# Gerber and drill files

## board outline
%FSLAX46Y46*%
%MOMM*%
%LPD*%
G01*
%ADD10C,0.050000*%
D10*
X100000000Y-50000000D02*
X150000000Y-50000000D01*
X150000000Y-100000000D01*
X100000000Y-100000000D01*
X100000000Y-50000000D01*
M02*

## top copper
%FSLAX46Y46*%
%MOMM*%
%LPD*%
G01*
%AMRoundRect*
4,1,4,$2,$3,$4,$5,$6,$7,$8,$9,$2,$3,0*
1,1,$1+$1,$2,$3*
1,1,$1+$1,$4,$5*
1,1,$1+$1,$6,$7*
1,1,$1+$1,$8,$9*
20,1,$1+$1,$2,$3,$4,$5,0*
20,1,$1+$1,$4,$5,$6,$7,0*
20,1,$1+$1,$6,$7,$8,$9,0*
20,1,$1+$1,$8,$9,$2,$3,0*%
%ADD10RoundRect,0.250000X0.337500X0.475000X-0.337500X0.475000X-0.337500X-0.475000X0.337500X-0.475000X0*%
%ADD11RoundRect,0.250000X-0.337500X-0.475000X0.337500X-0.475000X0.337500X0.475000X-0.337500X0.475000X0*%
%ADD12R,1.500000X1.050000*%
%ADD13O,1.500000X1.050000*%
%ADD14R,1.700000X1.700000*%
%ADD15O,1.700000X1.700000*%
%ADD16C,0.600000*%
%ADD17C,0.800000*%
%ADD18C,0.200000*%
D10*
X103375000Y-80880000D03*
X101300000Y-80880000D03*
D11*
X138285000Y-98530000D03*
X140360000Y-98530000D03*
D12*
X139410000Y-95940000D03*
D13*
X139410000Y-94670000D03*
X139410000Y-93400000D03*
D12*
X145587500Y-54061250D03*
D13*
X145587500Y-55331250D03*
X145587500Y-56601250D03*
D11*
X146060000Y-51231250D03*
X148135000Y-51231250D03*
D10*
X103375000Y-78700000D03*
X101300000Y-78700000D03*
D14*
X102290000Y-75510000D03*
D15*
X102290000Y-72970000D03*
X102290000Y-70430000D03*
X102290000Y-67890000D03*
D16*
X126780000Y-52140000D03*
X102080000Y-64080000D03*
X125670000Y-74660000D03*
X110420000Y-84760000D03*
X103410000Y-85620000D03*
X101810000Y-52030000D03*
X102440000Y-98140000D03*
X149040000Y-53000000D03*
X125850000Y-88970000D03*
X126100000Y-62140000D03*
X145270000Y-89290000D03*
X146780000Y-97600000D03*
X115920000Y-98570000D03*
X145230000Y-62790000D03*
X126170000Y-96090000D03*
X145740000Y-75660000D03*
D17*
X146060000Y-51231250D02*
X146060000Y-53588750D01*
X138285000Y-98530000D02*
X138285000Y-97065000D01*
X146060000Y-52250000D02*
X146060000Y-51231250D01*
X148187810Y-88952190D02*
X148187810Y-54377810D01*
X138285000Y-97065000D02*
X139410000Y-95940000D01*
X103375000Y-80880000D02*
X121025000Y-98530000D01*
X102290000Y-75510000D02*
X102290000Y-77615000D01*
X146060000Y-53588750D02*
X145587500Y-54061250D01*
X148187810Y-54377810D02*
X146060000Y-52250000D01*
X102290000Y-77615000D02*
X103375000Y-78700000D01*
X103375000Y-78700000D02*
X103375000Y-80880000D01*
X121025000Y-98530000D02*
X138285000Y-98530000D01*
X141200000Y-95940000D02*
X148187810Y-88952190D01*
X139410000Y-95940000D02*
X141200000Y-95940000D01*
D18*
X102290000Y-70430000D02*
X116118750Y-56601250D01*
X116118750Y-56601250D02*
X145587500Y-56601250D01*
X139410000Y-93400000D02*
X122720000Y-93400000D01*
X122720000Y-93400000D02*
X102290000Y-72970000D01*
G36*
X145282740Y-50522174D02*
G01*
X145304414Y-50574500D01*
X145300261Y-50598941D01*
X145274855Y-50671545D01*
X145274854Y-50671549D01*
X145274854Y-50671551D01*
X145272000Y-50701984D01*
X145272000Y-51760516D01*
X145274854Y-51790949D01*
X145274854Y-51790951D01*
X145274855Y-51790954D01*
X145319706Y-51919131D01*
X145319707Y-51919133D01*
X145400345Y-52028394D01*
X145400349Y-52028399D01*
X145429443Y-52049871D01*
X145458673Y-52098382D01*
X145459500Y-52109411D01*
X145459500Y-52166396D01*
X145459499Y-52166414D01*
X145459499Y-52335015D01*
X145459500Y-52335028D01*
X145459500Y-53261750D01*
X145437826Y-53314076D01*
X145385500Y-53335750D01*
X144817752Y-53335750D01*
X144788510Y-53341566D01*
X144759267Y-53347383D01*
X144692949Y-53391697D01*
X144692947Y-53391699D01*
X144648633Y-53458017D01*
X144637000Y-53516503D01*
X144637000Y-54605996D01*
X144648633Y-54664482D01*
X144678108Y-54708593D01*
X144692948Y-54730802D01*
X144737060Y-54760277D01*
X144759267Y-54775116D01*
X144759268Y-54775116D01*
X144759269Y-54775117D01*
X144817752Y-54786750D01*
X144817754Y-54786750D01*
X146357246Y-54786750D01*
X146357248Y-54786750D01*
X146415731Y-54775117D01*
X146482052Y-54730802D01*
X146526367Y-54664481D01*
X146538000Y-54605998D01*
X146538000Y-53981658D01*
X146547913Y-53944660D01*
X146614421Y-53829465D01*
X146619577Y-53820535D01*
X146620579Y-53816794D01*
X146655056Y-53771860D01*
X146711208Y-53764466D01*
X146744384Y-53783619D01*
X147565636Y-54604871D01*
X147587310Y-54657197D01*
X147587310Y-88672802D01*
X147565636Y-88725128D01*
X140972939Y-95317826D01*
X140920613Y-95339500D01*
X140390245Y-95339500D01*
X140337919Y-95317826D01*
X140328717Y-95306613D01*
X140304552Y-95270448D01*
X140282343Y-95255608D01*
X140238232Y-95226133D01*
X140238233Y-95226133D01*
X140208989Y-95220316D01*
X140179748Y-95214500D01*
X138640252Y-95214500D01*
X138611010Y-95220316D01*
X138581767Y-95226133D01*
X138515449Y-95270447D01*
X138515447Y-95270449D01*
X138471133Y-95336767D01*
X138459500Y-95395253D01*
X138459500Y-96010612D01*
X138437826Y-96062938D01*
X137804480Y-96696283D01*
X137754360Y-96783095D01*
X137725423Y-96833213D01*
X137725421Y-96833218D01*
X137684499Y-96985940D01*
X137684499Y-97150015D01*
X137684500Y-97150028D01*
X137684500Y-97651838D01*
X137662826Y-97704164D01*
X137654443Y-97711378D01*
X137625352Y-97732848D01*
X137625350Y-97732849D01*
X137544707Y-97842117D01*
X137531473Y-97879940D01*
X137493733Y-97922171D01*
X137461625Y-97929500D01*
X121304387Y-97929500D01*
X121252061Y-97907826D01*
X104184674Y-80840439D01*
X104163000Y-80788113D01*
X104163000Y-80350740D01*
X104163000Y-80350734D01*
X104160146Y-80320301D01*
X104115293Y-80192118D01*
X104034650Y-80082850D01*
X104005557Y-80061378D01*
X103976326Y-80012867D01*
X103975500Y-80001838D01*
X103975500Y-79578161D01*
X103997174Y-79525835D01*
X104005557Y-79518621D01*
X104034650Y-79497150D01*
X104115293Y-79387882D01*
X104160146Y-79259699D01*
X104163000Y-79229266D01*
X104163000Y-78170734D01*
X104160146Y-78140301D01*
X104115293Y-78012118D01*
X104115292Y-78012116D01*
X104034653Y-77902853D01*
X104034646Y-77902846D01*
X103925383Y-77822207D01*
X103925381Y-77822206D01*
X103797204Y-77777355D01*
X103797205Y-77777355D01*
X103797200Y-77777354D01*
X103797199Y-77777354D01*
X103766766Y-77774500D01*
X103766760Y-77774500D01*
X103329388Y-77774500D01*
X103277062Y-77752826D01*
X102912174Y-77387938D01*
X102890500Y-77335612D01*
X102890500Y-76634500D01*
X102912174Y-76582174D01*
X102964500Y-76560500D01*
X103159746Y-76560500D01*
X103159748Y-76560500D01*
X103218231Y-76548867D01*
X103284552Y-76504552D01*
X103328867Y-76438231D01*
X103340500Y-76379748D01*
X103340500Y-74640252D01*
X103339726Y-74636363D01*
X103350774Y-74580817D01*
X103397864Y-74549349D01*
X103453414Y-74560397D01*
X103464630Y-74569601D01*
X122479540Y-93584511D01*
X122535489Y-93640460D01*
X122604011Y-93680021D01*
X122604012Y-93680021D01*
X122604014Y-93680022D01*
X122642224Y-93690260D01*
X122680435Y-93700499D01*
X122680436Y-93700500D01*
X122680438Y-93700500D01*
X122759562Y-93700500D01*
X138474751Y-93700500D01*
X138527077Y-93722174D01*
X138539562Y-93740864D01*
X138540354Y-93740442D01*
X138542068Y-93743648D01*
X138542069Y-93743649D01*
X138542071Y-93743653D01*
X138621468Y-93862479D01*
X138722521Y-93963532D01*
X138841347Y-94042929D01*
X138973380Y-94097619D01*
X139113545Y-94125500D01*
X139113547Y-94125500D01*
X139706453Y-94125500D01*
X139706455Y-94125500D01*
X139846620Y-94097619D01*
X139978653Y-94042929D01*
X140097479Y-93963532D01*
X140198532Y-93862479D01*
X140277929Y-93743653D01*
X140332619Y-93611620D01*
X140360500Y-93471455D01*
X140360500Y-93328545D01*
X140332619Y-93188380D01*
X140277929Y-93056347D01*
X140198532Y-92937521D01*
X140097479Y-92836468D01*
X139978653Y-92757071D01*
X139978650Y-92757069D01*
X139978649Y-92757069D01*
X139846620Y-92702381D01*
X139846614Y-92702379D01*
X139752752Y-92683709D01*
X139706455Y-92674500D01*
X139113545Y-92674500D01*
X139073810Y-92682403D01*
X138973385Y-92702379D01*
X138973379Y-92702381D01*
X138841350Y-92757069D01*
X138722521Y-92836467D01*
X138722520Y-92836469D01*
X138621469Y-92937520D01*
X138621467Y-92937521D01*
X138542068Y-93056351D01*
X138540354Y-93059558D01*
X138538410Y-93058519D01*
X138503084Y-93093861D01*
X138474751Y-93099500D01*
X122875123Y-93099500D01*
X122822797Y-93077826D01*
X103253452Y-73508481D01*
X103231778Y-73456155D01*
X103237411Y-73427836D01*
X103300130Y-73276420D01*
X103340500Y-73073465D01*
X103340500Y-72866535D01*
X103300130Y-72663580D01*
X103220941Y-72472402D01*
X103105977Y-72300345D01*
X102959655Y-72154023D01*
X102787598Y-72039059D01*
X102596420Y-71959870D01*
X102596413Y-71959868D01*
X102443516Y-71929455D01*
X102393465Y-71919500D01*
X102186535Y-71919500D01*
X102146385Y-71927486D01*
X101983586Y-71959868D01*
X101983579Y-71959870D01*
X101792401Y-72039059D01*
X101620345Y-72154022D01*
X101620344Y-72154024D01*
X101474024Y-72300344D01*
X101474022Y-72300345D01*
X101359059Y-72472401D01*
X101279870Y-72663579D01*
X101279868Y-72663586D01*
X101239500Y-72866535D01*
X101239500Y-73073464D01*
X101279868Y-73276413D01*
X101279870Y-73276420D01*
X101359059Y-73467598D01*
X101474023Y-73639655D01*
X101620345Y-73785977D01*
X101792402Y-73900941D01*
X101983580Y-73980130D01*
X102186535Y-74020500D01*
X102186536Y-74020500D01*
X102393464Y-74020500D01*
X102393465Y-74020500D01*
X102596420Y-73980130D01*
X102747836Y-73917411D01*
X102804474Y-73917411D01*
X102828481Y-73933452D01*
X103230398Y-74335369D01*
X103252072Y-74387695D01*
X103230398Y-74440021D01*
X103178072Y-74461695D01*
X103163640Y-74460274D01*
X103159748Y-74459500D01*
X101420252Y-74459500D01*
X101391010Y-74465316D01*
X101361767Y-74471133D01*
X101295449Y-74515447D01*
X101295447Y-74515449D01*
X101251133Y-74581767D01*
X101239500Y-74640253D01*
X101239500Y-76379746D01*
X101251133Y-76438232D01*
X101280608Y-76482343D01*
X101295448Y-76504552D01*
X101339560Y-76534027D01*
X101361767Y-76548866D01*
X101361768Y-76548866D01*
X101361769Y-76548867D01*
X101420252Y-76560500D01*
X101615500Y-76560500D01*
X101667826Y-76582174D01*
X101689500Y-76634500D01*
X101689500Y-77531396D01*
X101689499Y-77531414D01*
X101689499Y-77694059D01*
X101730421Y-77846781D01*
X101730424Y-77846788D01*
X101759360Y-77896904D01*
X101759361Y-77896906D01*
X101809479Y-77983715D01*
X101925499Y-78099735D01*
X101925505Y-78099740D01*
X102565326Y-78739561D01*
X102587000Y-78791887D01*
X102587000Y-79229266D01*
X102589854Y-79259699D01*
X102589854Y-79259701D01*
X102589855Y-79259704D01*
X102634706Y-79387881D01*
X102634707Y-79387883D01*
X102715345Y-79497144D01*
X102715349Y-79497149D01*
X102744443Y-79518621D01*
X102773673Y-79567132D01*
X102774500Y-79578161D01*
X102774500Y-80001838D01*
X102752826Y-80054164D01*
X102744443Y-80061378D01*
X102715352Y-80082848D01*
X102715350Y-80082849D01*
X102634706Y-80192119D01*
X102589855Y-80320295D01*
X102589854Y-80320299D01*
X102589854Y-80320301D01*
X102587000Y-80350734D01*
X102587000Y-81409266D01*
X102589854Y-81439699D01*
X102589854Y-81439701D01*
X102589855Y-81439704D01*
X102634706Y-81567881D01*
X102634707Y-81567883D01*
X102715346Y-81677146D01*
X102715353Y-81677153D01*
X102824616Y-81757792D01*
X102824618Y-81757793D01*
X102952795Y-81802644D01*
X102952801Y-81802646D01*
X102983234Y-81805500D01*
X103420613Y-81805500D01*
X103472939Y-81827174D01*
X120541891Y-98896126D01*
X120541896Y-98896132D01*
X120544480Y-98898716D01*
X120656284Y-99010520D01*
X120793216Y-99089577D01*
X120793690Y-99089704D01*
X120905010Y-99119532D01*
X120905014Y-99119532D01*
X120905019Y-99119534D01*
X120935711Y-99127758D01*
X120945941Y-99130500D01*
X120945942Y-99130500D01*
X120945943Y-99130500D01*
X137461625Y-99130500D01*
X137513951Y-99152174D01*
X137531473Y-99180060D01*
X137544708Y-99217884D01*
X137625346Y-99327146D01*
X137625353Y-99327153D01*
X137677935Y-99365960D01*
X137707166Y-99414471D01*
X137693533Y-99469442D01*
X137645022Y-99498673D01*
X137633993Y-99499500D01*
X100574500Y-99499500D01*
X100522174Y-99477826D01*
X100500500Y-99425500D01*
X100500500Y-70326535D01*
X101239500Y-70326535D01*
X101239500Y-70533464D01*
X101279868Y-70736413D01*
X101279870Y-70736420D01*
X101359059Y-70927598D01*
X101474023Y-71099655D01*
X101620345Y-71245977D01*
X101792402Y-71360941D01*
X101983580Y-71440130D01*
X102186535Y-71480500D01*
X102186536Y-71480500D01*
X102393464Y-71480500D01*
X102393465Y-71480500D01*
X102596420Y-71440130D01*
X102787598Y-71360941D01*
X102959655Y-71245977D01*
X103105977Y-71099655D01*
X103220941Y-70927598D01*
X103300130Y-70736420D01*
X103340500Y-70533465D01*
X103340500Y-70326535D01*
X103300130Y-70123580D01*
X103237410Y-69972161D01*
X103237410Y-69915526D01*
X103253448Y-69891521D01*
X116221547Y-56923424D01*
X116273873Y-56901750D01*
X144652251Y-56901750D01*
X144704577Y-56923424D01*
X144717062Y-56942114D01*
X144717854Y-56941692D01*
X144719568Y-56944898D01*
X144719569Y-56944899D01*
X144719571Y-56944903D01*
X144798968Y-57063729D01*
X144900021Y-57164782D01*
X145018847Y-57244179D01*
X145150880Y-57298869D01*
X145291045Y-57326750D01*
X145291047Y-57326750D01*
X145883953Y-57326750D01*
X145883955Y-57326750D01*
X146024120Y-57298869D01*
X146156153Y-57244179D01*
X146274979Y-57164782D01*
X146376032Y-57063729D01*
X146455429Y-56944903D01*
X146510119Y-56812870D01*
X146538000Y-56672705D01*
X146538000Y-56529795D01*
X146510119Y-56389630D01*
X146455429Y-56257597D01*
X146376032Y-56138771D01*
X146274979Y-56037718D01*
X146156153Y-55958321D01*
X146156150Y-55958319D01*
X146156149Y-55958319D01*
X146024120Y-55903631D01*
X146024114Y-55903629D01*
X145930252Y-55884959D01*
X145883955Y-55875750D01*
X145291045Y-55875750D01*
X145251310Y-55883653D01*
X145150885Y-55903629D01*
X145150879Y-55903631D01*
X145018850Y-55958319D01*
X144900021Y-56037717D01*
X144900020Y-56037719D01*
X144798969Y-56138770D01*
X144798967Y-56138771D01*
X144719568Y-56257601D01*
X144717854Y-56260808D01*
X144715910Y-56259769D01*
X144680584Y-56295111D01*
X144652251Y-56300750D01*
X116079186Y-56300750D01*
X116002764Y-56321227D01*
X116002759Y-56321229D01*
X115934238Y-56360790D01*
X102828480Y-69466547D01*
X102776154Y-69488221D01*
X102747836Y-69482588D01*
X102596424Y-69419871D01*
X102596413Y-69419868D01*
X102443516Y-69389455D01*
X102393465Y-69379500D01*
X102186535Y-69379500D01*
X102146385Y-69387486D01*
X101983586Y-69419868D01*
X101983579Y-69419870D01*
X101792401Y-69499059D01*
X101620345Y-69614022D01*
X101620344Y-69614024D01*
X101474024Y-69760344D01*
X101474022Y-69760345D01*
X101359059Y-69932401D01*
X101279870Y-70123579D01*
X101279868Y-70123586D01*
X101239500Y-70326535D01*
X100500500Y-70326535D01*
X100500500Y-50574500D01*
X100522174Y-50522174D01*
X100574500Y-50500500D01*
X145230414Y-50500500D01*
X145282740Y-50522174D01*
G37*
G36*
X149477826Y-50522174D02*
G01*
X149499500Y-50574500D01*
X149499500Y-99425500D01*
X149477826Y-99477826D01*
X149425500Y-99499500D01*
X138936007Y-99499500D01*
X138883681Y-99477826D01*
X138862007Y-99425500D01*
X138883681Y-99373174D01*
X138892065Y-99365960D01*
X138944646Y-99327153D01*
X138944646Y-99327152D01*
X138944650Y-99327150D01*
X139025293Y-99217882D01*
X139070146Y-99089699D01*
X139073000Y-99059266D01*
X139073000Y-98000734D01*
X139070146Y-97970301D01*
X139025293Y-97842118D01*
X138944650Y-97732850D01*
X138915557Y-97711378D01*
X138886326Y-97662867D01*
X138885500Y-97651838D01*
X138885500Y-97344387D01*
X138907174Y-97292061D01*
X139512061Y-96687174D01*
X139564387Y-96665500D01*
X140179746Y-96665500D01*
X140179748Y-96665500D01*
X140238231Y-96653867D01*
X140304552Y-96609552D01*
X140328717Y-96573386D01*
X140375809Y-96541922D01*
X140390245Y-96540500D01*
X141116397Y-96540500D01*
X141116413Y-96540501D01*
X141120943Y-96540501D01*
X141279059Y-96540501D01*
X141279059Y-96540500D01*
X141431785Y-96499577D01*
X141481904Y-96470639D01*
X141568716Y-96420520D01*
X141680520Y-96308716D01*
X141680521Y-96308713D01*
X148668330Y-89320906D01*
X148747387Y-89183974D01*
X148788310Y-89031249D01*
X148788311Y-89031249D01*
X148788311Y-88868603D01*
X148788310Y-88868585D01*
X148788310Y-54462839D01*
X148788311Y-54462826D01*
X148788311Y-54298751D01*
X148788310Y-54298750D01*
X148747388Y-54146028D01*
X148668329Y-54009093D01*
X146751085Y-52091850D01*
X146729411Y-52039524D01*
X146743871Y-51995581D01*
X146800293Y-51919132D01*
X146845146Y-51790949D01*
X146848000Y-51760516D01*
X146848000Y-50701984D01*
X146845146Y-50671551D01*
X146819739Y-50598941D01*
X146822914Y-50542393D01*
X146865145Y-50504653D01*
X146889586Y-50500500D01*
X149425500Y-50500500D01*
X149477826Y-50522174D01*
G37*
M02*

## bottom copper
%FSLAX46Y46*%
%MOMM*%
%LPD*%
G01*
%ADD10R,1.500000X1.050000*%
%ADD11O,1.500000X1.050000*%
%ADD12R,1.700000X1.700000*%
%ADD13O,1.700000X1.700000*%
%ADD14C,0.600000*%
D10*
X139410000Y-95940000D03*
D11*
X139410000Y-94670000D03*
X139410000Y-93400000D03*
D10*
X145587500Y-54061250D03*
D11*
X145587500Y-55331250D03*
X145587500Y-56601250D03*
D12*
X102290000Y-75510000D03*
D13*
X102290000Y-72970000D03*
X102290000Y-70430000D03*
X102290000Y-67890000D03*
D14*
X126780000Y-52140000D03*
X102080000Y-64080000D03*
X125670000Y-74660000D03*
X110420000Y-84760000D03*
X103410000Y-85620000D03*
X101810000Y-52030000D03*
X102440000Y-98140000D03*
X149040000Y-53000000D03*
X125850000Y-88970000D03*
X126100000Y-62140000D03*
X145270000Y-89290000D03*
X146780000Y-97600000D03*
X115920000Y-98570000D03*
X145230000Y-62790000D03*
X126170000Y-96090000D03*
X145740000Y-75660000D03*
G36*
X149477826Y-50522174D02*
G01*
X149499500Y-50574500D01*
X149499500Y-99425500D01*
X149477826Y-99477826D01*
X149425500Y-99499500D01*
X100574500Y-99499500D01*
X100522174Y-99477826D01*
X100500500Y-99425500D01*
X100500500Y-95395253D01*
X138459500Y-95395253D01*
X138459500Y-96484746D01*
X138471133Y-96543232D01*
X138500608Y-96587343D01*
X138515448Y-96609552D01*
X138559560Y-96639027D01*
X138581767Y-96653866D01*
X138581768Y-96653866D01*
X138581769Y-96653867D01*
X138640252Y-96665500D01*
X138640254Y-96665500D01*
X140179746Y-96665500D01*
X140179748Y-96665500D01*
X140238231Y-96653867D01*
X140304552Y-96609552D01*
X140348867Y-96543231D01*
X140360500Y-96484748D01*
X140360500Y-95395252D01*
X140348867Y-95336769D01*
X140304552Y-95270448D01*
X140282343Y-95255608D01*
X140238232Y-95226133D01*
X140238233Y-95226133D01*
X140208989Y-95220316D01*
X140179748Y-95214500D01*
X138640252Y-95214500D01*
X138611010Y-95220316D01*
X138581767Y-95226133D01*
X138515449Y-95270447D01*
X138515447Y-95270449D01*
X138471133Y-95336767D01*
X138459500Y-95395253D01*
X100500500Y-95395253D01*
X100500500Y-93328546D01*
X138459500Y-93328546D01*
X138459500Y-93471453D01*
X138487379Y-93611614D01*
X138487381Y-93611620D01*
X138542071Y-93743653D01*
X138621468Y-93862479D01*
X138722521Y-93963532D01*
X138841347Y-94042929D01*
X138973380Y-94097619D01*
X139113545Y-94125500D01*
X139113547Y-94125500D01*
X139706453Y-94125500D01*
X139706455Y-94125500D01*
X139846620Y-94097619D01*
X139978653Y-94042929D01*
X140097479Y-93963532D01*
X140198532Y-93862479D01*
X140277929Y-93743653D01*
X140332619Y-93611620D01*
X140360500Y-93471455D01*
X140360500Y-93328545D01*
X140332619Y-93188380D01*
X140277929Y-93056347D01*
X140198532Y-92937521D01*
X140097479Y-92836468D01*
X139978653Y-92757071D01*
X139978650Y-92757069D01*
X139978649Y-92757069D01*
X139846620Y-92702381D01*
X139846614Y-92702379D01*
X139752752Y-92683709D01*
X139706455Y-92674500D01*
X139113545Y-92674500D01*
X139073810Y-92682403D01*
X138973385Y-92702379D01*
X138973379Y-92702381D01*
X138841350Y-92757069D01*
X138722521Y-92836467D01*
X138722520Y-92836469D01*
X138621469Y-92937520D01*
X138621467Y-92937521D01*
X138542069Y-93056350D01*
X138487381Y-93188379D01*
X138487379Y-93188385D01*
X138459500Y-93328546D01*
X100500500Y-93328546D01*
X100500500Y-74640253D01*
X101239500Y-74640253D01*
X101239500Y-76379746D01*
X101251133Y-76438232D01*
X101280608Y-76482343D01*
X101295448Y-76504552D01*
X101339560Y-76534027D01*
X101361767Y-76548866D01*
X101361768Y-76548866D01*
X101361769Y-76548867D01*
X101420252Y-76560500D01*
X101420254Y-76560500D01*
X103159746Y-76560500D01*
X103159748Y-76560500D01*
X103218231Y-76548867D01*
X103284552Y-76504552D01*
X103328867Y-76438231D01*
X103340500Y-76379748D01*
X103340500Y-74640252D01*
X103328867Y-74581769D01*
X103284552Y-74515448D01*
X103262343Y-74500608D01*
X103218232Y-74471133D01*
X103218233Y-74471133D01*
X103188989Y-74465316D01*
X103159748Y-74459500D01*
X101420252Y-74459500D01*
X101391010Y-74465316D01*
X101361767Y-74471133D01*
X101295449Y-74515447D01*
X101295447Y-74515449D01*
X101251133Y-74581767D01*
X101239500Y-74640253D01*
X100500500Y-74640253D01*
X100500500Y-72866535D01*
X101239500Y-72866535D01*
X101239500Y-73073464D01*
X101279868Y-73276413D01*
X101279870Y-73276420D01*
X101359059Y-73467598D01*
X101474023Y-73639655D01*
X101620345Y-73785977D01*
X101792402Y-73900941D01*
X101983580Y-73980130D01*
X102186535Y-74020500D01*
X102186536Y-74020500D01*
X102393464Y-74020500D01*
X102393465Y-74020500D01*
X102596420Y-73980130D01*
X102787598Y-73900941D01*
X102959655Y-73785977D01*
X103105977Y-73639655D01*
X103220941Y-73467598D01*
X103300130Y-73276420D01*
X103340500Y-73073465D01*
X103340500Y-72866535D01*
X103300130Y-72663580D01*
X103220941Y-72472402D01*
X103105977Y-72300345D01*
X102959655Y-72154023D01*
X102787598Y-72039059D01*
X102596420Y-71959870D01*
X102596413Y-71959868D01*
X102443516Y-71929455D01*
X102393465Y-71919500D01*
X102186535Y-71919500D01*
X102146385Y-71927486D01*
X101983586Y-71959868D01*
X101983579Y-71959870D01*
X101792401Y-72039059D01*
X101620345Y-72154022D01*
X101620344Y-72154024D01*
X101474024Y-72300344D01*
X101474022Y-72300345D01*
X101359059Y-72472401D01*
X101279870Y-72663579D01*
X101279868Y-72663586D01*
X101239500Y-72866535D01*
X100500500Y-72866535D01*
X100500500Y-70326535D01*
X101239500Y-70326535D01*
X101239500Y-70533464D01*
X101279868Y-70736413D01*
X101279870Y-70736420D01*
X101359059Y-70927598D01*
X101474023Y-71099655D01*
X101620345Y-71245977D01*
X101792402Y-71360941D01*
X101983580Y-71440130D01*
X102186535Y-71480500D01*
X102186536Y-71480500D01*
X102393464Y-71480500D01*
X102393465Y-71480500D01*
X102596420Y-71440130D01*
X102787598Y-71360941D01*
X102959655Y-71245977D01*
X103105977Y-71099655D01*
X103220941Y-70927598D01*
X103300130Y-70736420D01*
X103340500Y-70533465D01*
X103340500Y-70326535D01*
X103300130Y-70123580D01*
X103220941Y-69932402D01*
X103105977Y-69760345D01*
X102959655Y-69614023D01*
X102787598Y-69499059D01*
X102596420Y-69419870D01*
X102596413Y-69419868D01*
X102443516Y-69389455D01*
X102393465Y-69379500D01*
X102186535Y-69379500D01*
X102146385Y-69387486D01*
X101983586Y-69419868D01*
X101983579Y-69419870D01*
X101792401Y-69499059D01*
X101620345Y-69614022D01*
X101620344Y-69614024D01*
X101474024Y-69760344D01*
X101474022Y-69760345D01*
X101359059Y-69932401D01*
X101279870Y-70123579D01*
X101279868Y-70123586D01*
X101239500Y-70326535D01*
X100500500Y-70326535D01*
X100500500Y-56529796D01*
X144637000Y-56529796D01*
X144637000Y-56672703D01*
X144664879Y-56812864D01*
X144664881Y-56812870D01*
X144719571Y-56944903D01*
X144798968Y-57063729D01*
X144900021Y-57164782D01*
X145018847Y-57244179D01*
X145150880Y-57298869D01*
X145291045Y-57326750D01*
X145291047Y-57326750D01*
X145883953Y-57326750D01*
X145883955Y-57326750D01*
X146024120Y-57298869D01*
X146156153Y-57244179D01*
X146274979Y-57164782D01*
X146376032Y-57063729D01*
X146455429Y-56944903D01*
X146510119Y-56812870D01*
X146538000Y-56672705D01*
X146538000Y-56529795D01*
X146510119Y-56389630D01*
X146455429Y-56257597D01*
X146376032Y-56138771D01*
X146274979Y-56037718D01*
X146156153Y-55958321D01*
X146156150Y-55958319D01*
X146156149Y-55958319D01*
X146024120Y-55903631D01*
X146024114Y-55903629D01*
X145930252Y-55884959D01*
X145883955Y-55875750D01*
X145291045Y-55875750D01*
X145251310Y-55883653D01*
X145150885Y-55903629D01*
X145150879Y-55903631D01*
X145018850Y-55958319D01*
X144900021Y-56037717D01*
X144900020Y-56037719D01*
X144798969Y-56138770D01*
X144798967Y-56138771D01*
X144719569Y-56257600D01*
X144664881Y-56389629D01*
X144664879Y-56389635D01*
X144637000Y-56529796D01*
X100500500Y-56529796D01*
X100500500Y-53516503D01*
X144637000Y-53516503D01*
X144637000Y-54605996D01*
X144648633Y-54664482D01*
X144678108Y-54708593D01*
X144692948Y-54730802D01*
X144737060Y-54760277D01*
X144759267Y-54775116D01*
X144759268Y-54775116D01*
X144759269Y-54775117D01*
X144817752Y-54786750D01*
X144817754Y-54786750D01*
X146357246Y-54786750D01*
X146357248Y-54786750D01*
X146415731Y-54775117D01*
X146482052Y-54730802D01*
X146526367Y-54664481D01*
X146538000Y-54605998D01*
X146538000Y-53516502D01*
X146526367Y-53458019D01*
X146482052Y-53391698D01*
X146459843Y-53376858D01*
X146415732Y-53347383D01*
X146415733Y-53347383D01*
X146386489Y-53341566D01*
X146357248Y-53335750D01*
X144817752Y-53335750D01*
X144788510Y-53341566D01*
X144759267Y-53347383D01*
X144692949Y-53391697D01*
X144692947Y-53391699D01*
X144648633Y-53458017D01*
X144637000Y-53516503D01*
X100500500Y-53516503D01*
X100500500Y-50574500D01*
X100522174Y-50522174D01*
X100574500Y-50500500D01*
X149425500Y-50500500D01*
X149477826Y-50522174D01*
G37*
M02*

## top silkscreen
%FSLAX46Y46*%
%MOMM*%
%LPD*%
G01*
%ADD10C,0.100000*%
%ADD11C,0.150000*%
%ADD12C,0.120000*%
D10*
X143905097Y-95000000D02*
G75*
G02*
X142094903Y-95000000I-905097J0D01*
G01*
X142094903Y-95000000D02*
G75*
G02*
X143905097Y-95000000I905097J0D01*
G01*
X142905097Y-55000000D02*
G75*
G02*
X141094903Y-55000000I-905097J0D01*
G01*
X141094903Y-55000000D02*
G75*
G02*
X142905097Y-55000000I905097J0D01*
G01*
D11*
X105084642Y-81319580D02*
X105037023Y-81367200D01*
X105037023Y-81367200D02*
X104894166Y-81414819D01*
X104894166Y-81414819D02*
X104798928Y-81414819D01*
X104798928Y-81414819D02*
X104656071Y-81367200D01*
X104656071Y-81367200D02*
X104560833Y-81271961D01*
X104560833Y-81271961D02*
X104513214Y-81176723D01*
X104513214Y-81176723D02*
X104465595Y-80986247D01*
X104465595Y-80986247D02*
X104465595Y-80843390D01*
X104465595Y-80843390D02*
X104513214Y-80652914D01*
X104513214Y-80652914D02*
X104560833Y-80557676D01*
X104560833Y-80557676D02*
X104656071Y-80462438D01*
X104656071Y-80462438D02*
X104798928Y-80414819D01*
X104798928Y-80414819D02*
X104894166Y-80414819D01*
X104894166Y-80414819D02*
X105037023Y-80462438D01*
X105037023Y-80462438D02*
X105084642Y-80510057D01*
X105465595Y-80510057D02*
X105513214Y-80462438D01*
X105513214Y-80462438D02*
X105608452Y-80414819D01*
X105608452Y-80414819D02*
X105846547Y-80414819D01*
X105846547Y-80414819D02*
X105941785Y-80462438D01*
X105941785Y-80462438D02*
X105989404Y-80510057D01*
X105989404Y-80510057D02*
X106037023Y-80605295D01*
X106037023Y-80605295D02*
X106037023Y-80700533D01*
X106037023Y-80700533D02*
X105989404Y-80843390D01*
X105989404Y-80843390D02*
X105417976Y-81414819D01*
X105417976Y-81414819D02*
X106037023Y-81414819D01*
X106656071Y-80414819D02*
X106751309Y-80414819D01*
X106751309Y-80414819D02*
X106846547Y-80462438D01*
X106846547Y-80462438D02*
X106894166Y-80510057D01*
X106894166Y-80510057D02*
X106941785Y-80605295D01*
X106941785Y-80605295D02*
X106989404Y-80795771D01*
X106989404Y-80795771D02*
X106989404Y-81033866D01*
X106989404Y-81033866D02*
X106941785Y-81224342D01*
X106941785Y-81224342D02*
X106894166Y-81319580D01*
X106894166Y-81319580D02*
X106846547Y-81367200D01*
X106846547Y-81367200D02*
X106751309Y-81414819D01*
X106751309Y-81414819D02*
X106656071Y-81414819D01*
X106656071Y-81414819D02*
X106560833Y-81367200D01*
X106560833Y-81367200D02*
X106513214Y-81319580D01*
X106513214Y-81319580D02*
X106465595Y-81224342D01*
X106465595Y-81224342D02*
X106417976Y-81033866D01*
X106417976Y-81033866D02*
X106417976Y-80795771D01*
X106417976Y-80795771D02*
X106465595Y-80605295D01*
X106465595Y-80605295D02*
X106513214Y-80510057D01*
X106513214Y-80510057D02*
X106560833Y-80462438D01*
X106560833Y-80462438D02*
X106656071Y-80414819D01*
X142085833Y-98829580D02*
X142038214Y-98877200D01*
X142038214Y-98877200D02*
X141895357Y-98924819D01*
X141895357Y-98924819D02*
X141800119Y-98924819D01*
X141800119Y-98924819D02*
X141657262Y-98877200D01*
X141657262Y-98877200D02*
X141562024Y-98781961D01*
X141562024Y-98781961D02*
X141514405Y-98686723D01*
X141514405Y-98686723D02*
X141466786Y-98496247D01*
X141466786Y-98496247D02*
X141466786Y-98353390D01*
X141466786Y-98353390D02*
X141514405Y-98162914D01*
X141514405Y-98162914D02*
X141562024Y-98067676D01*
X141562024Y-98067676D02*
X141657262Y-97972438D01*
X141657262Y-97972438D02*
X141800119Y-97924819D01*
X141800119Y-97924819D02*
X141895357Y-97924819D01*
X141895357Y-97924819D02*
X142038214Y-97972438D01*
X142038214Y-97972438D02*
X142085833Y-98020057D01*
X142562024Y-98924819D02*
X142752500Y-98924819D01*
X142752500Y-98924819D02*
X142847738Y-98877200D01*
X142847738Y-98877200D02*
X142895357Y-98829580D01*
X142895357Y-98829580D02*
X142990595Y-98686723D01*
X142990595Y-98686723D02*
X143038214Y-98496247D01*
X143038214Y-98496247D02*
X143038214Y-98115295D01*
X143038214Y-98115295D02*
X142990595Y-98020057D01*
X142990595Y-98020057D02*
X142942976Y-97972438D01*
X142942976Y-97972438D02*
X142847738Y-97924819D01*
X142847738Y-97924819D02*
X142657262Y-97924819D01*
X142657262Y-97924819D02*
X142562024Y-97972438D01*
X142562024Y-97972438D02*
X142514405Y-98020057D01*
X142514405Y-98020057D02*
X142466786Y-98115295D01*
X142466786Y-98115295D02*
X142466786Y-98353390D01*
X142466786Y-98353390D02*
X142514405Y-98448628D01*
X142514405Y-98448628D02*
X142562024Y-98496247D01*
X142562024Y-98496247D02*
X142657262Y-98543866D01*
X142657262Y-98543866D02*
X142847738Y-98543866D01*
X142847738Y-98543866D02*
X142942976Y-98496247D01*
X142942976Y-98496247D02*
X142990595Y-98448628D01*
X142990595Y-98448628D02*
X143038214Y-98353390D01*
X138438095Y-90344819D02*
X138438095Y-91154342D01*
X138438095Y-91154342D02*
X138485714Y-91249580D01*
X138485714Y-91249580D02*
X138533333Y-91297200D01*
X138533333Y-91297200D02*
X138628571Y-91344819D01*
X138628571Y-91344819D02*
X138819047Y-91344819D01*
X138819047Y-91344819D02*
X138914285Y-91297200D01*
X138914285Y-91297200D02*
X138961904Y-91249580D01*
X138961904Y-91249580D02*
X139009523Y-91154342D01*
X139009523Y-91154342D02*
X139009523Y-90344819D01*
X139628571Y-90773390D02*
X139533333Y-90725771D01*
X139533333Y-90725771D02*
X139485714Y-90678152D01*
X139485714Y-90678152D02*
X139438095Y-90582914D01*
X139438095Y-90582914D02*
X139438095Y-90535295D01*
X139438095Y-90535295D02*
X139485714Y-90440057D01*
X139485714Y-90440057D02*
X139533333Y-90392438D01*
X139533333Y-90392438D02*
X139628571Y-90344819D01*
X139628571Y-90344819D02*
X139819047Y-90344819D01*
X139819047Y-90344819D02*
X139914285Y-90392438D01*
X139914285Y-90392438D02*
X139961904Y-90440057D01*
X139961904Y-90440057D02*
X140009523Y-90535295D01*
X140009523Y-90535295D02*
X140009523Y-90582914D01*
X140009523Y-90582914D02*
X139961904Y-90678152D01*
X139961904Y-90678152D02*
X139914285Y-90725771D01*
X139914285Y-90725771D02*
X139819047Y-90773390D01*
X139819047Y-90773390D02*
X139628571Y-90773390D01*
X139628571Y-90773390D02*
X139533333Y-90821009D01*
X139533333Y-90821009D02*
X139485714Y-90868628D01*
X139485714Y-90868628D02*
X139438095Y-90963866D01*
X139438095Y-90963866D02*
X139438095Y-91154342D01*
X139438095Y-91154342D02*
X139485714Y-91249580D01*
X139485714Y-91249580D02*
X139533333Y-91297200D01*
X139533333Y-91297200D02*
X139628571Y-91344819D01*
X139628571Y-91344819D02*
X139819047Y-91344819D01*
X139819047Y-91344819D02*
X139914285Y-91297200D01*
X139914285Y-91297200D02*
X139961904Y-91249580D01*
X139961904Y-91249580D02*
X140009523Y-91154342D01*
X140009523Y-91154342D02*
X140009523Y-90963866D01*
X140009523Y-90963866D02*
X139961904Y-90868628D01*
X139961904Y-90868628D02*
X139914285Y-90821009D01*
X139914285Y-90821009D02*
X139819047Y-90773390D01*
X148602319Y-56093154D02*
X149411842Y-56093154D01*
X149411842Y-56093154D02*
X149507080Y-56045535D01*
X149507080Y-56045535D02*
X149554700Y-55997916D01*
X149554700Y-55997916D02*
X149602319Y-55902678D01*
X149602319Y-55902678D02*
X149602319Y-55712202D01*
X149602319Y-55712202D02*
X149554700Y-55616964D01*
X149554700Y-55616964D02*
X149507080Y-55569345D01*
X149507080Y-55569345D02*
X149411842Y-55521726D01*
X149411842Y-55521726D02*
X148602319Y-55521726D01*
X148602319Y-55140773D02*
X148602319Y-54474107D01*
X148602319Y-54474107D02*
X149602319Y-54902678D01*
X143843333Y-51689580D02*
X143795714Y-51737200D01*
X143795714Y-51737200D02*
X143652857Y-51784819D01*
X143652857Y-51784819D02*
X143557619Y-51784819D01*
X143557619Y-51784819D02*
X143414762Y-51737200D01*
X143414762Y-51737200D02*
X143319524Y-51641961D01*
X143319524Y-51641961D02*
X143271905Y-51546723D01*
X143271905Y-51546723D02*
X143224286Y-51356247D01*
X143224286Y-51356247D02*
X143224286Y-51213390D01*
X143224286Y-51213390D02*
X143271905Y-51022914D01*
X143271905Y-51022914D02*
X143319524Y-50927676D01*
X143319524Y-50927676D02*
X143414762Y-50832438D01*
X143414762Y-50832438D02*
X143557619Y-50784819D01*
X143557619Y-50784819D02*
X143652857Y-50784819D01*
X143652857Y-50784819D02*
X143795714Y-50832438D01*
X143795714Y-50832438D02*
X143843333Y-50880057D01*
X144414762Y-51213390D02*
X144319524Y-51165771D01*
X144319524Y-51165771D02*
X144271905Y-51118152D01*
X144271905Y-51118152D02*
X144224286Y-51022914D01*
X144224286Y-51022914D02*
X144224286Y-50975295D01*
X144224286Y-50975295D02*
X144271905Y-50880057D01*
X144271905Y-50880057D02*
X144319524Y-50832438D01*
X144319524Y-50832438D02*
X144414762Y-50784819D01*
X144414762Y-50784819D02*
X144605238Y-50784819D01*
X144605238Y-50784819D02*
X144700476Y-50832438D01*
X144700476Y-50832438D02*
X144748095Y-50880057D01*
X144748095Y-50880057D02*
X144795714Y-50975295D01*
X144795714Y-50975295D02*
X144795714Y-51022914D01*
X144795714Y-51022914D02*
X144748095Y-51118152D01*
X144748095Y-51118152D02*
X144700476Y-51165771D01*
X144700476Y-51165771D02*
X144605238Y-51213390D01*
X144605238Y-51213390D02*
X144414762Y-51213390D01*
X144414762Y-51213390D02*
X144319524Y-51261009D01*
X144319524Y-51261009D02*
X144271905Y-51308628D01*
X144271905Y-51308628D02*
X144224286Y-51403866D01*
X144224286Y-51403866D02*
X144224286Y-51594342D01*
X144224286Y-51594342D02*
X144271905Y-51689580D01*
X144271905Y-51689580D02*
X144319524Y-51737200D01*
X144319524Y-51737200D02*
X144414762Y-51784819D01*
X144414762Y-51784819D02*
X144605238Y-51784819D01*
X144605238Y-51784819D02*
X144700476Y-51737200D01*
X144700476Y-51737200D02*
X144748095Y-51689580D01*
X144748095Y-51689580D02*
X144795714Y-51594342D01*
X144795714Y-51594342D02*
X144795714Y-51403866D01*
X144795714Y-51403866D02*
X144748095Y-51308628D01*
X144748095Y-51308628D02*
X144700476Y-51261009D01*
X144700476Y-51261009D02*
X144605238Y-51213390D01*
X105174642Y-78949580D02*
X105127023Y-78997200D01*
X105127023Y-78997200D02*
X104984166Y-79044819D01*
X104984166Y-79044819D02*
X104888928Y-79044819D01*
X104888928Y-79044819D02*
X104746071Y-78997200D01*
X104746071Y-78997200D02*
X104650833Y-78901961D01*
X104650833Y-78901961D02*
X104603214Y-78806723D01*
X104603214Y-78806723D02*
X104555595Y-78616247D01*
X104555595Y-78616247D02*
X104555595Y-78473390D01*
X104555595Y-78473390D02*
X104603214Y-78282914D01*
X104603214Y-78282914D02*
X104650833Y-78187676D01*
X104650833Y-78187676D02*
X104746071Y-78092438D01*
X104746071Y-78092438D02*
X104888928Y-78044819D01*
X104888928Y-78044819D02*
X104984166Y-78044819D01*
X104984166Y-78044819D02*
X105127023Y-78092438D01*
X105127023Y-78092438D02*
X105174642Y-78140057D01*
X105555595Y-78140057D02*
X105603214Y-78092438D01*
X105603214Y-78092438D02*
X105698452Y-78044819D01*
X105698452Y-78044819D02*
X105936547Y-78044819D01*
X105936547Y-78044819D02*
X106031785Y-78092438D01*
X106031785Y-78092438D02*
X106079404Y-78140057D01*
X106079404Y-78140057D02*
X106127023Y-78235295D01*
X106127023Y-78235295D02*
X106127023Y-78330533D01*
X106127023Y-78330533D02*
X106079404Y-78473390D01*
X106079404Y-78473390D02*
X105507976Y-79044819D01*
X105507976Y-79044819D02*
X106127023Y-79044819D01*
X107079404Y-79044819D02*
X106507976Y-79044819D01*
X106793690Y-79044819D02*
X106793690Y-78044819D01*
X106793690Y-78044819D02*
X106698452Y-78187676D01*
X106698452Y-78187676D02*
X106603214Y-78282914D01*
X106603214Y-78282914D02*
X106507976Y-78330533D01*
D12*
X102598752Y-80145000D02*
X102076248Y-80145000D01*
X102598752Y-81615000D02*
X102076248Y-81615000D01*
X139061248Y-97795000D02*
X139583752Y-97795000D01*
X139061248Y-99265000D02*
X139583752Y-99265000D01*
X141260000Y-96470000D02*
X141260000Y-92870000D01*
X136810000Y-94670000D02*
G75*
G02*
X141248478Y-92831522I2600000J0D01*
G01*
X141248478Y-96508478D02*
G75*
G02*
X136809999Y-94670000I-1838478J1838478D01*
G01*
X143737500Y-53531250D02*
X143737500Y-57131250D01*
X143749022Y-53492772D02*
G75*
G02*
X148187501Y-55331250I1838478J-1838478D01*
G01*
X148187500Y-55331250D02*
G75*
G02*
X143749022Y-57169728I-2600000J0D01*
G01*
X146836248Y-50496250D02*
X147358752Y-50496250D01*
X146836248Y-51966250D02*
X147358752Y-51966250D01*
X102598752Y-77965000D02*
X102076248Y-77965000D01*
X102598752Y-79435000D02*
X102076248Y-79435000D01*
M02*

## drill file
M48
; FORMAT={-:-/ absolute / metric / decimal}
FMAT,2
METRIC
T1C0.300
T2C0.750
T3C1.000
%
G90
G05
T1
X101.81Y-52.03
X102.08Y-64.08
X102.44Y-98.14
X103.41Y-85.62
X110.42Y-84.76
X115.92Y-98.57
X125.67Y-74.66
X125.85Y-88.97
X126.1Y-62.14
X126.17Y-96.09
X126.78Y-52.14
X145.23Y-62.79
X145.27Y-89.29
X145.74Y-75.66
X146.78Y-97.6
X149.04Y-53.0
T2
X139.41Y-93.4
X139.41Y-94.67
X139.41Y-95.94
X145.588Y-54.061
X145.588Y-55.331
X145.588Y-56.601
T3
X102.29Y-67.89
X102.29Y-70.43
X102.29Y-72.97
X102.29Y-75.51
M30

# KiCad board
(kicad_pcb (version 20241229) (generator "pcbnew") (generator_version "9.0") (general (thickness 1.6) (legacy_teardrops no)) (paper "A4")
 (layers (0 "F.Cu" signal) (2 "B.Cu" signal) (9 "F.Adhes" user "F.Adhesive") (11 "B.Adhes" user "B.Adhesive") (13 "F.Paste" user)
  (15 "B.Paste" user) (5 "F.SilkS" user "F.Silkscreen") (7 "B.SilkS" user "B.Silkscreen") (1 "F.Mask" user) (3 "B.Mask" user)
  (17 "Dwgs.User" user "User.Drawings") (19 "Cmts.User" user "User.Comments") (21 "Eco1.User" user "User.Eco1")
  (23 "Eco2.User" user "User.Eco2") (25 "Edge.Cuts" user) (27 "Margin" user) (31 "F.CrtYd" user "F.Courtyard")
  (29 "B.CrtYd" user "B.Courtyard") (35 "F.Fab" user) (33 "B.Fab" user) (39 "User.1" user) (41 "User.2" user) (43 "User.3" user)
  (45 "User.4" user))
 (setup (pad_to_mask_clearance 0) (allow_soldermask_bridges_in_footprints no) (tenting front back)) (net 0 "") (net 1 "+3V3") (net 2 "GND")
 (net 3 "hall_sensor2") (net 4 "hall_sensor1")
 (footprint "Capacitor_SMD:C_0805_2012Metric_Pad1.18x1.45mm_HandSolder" (layer "F.Cu") (at 102.3375 80.88 180)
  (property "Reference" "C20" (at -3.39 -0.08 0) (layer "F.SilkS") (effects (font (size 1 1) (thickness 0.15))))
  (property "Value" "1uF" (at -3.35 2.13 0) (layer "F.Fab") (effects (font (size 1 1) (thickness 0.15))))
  (fp_line (start -0.261252 0.735) (end 0.261252 0.735) (stroke (width 0.12) (type solid)) (layer "F.SilkS"))
  (fp_line (start -0.261252 -0.735) (end 0.261252 -0.735) (stroke (width 0.12) (type solid)) (layer "F.SilkS"))
  (pad "1" smd roundrect (at -1.0375 0 180) (size 1.175 1.45) (layers "F.Cu" "F.Mask" "F.Paste") (roundrect_rratio 0.212766) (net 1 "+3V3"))
  (pad "2" smd roundrect (at 1.0375 0 180) (size 1.175 1.45) (layers "F.Cu" "F.Mask" "F.Paste") (roundrect_rratio 0.212766) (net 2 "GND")))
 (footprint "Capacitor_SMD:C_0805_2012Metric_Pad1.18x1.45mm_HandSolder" (layer "F.Cu") (at 139.3225 98.53)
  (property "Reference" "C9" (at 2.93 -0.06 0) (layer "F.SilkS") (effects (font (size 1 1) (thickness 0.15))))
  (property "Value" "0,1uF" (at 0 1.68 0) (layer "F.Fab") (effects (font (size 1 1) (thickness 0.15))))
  (fp_line (start -0.261252 -0.735) (end 0.261252 -0.735) (stroke (width 0.12) (type solid)) (layer "F.SilkS"))
  (fp_line (start -0.261252 0.735) (end 0.261252 0.735) (stroke (width 0.12) (type solid)) (layer "F.SilkS"))
  (pad "1" smd roundrect (at -1.0375 0) (size 1.175 1.45) (layers "F.Cu" "F.Mask" "F.Paste") (roundrect_rratio 0.212766) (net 1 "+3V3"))
  (pad "2" smd roundrect (at 1.0375 0) (size 1.175 1.45) (layers "F.Cu" "F.Mask" "F.Paste") (roundrect_rratio 0.212766) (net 2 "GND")))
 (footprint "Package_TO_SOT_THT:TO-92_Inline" (layer "F.Cu") (at 139.41 95.94 90)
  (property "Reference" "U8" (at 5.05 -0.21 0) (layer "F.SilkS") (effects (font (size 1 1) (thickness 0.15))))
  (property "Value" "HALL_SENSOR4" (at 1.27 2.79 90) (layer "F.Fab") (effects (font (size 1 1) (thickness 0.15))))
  (fp_line (start -0.53 1.85) (end 3.07 1.85) (stroke (width 0.12) (type solid)) (layer "F.SilkS"))
  (fp_arc (start 1.27 -2.6) (mid 3.672087 -0.994977) (end 3.108478 1.838478) (stroke (width 0.12) (type solid)) (layer "F.SilkS"))
  (fp_arc (start -0.568478 1.838478) (mid -1.132087 -0.994977) (end 1.27 -2.6) (stroke (width 0.12) (type solid)) (layer "F.SilkS"))
  (pad "1" thru_hole rect (at 0 0 90) (size 1.05 1.5) (drill 0.75) (layers "*.Cu" "*.Mask") (remove_unused_layers no) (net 1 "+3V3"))
  (pad "2" thru_hole oval (at 1.27 0 90) (size 1.05 1.5) (drill 0.75) (layers "*.Cu" "*.Mask") (remove_unused_layers no) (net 2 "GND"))
  (pad "3" thru_hole oval (at 2.54 0 90) (size 1.05 1.5) (drill 0.75) (layers "*.Cu" "*.Mask") (remove_unused_layers no)
   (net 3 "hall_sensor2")))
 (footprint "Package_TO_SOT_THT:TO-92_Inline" (layer "F.Cu") (at 145.5875 54.06125 -90)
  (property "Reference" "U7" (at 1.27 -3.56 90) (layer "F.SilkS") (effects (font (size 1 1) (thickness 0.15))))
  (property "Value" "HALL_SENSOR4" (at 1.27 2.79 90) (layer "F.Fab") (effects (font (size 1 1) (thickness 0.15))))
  (fp_line (start -0.53 1.85) (end 3.07 1.85) (stroke (width 0.12) (type solid)) (layer "F.SilkS"))
  (fp_arc (start -0.568478 1.838478) (mid -1.132087 -0.994977) (end 1.27 -2.6) (stroke (width 0.12) (type solid)) (layer "F.SilkS"))
  (fp_arc (start 1.27 -2.6) (mid 3.672087 -0.994977) (end 3.108478 1.838478) (stroke (width 0.12) (type solid)) (layer "F.SilkS"))
  (pad "1" thru_hole rect (at 0 0 270) (size 1.05 1.5) (drill 0.75) (layers "*.Cu" "*.Mask") (remove_unused_layers no) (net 1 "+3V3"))
  (pad "2" thru_hole oval (at 1.27 0 270) (size 1.05 1.5) (drill 0.75) (layers "*.Cu" "*.Mask") (remove_unused_layers no) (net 2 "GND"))
  (pad "3" thru_hole oval (at 2.54 0 270) (size 1.05 1.5) (drill 0.75) (layers "*.Cu" "*.Mask") (remove_unused_layers no)
   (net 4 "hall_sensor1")))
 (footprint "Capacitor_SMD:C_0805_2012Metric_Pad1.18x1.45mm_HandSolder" (layer "F.Cu") (at 147.0975 51.23125)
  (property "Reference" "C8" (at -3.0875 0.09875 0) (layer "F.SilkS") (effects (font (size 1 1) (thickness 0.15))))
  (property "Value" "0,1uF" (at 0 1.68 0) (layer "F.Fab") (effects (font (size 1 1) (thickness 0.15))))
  (fp_line (start -0.261252 -0.735) (end 0.261252 -0.735) (stroke (width 0.12) (type solid)) (layer "F.SilkS"))
  (fp_line (start -0.261252 0.735) (end 0.261252 0.735) (stroke (width 0.12) (type solid)) (layer "F.SilkS"))
  (pad "1" smd roundrect (at -1.0375 0) (size 1.175 1.45) (layers "F.Cu" "F.Mask" "F.Paste") (roundrect_rratio 0.212766) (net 1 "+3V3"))
  (pad "2" smd roundrect (at 1.0375 0) (size 1.175 1.45) (layers "F.Cu" "F.Mask" "F.Paste") (roundrect_rratio 0.212766) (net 2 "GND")))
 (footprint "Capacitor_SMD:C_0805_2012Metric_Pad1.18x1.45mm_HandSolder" (layer "F.Cu") (at 102.3375 78.7 180)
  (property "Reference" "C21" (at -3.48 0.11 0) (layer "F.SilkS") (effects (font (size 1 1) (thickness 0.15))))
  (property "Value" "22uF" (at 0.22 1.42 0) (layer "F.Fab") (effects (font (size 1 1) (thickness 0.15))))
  (fp_line (start -0.261252 0.735) (end 0.261252 0.735) (stroke (width 0.12) (type solid)) (layer "F.SilkS"))
  (fp_line (start -0.261252 -0.735) (end 0.261252 -0.735) (stroke (width 0.12) (type solid)) (layer "F.SilkS"))
  (pad "1" smd roundrect (at -1.0375 0 180) (size 1.175 1.45) (layers "F.Cu" "F.Mask" "F.Paste") (roundrect_rratio 0.212766) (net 1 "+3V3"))
  (pad "2" smd roundrect (at 1.0375 0 180) (size 1.175 1.45) (layers "F.Cu" "F.Mask" "F.Paste") (roundrect_rratio 0.212766) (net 2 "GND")))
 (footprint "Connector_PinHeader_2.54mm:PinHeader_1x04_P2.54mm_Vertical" (layer "B.Cu") (at 102.29 75.51)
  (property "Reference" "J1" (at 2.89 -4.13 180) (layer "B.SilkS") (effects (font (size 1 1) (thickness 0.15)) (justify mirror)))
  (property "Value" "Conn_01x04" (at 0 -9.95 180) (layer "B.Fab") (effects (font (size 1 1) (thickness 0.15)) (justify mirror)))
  (pad "1" thru_hole rect (at 0 0) (size 1.7 1.7) (drill 1) (layers "*.Cu" "*.Mask") (remove_unused_layers no) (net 1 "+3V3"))
  (pad "2" thru_hole oval (at 0 -2.54) (size 1.7 1.7) (drill 1) (layers "*.Cu" "*.Mask") (remove_unused_layers no) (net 3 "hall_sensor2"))
  (pad "3" thru_hole oval (at 0 -5.08) (size 1.7 1.7) (drill 1) (layers "*.Cu" "*.Mask") (remove_unused_layers no) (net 4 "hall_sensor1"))
  (pad "4" thru_hole oval (at 0 -7.62) (size 1.7 1.7) (drill 1) (layers "*.Cu" "*.Mask") (remove_unused_layers no) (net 2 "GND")))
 (gr_circle (center 143 95) (end 143.905097 95) (stroke (width 0.1) (type solid)) (fill no) (layer "F.SilkS"))
 (gr_circle (center 142 55) (end 142.905097 55) (stroke (width 0.1) (type solid)) (fill no) (layer "F.SilkS"))
 (gr_rect (start 100 50) (end 150 100) (stroke (width 0.05) (type solid)) (fill no) (layer "Edge.Cuts"))
 (via (at 126.78 52.14) (size 0.6) (drill 0.3) (layers "F.Cu" "B.Cu") (free yes) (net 2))
 (via (at 102.08 64.08) (size 0.6) (drill 0.3) (layers "F.Cu" "B.Cu") (free yes) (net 2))
 (via (at 125.67 74.66) (size 0.6) (drill 0.3) (layers "F.Cu" "B.Cu") (free yes) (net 2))
 (via (at 110.42 84.76) (size 0.6) (drill 0.3) (layers "F.Cu" "B.Cu") (free yes) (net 2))
 (via (at 103.41 85.62) (size 0.6) (drill 0.3) (layers "F.Cu" "B.Cu") (free yes) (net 2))
 (via (at 101.81 52.03) (size 0.6) (drill 0.3) (layers "F.Cu" "B.Cu") (free yes) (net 2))
 (via (at 102.44 98.14) (size 0.6) (drill 0.3) (layers "F.Cu" "B.Cu") (free yes) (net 2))
 (via (at 149.04 53) (size 0.6) (drill 0.3) (layers "F.Cu" "B.Cu") (free yes) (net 2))
 (via (at 125.85 88.97) (size 0.6) (drill 0.3) (layers "F.Cu" "B.Cu") (free yes) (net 2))
 (via (at 126.1 62.14) (size 0.6) (drill 0.3) (layers "F.Cu" "B.Cu") (free yes) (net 2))
 (via (at 145.27 89.29) (size 0.6) (drill 0.3) (layers "F.Cu" "B.Cu") (free yes) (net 2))
 (via (at 146.78 97.6) (size 0.6) (drill 0.3) (layers "F.Cu" "B.Cu") (free yes) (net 2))
 (via (at 115.92 98.57) (size 0.6) (drill 0.3) (layers "F.Cu" "B.Cu") (free yes) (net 2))
 (via (at 145.23 62.79) (size 0.6) (drill 0.3) (layers "F.Cu" "B.Cu") (free yes) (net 2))
 (via (at 126.17 96.09) (size 0.6) (drill 0.3) (layers "F.Cu" "B.Cu") (free yes) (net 2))
 (via (at 145.74 75.66) (size 0.6) (drill 0.3) (layers "F.Cu" "B.Cu") (free yes) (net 2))
 (segment (start 146.06 51.23125) (end 146.06 53.58875) (width 0.8) (layer "F.Cu") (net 1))
 (segment (start 138.285 98.53) (end 138.285 97.065) (width 0.8) (layer "F.Cu") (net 1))
 (segment (start 146.06 52.25) (end 146.06 51.23125) (width 0.8) (layer "F.Cu") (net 1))
 (segment (start 148.18781 88.95219) (end 148.18781 54.37781) (width 0.8) (layer "F.Cu") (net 1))
 (segment (start 138.285 97.065) (end 139.41 95.94) (width 0.8) (layer "F.Cu") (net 1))
 (segment (start 103.375 80.88) (end 121.025 98.53) (width 0.8) (layer "F.Cu") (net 1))
 (segment (start 102.29 75.51) (end 102.29 77.615) (width 0.8) (layer "F.Cu") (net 1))
 (segment (start 146.06 53.58875) (end 145.5875 54.06125) (width 0.8) (layer "F.Cu") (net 1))
 (segment (start 148.18781 54.37781) (end 146.06 52.25) (width 0.8) (layer "F.Cu") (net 1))
 (segment (start 102.29 77.615) (end 103.375 78.7) (width 0.8) (layer "F.Cu") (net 1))
 (segment (start 103.375 78.7) (end 103.375 80.88) (width 0.8) (layer "F.Cu") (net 1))
 (segment (start 121.025 98.53) (end 138.285 98.53) (width 0.8) (layer "F.Cu") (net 1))
 (segment (start 141.2 95.94) (end 148.18781 88.95219) (width 0.8) (layer "F.Cu") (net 1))
 (segment (start 139.41 95.94) (end 141.2 95.94) (width 0.8) (layer "F.Cu") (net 1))
 (segment (start 102.29 70.43) (end 116.11875 56.60125) (width 0.2) (layer "F.Cu") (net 4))
 (segment (start 116.11875 56.60125) (end 145.5875 56.60125) (width 0.2) (layer "F.Cu") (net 4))
 (segment (start 139.41 93.4) (end 122.72 93.4) (width 0.2) (layer "F.Cu") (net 3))
 (segment (start 122.72 93.4) (end 102.29 72.97) (width 0.2) (layer "F.Cu") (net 3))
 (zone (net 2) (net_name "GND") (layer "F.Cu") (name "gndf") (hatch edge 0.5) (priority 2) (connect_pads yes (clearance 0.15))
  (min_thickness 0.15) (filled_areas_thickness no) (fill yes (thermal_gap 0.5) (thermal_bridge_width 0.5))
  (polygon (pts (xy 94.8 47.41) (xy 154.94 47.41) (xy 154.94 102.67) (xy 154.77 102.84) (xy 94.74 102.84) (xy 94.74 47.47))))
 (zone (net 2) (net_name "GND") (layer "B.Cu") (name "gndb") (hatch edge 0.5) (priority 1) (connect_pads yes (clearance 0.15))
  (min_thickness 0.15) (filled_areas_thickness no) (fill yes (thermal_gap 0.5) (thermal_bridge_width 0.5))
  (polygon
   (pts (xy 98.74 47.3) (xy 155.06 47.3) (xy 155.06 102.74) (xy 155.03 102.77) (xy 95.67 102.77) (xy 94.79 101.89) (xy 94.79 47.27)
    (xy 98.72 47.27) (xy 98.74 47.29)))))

